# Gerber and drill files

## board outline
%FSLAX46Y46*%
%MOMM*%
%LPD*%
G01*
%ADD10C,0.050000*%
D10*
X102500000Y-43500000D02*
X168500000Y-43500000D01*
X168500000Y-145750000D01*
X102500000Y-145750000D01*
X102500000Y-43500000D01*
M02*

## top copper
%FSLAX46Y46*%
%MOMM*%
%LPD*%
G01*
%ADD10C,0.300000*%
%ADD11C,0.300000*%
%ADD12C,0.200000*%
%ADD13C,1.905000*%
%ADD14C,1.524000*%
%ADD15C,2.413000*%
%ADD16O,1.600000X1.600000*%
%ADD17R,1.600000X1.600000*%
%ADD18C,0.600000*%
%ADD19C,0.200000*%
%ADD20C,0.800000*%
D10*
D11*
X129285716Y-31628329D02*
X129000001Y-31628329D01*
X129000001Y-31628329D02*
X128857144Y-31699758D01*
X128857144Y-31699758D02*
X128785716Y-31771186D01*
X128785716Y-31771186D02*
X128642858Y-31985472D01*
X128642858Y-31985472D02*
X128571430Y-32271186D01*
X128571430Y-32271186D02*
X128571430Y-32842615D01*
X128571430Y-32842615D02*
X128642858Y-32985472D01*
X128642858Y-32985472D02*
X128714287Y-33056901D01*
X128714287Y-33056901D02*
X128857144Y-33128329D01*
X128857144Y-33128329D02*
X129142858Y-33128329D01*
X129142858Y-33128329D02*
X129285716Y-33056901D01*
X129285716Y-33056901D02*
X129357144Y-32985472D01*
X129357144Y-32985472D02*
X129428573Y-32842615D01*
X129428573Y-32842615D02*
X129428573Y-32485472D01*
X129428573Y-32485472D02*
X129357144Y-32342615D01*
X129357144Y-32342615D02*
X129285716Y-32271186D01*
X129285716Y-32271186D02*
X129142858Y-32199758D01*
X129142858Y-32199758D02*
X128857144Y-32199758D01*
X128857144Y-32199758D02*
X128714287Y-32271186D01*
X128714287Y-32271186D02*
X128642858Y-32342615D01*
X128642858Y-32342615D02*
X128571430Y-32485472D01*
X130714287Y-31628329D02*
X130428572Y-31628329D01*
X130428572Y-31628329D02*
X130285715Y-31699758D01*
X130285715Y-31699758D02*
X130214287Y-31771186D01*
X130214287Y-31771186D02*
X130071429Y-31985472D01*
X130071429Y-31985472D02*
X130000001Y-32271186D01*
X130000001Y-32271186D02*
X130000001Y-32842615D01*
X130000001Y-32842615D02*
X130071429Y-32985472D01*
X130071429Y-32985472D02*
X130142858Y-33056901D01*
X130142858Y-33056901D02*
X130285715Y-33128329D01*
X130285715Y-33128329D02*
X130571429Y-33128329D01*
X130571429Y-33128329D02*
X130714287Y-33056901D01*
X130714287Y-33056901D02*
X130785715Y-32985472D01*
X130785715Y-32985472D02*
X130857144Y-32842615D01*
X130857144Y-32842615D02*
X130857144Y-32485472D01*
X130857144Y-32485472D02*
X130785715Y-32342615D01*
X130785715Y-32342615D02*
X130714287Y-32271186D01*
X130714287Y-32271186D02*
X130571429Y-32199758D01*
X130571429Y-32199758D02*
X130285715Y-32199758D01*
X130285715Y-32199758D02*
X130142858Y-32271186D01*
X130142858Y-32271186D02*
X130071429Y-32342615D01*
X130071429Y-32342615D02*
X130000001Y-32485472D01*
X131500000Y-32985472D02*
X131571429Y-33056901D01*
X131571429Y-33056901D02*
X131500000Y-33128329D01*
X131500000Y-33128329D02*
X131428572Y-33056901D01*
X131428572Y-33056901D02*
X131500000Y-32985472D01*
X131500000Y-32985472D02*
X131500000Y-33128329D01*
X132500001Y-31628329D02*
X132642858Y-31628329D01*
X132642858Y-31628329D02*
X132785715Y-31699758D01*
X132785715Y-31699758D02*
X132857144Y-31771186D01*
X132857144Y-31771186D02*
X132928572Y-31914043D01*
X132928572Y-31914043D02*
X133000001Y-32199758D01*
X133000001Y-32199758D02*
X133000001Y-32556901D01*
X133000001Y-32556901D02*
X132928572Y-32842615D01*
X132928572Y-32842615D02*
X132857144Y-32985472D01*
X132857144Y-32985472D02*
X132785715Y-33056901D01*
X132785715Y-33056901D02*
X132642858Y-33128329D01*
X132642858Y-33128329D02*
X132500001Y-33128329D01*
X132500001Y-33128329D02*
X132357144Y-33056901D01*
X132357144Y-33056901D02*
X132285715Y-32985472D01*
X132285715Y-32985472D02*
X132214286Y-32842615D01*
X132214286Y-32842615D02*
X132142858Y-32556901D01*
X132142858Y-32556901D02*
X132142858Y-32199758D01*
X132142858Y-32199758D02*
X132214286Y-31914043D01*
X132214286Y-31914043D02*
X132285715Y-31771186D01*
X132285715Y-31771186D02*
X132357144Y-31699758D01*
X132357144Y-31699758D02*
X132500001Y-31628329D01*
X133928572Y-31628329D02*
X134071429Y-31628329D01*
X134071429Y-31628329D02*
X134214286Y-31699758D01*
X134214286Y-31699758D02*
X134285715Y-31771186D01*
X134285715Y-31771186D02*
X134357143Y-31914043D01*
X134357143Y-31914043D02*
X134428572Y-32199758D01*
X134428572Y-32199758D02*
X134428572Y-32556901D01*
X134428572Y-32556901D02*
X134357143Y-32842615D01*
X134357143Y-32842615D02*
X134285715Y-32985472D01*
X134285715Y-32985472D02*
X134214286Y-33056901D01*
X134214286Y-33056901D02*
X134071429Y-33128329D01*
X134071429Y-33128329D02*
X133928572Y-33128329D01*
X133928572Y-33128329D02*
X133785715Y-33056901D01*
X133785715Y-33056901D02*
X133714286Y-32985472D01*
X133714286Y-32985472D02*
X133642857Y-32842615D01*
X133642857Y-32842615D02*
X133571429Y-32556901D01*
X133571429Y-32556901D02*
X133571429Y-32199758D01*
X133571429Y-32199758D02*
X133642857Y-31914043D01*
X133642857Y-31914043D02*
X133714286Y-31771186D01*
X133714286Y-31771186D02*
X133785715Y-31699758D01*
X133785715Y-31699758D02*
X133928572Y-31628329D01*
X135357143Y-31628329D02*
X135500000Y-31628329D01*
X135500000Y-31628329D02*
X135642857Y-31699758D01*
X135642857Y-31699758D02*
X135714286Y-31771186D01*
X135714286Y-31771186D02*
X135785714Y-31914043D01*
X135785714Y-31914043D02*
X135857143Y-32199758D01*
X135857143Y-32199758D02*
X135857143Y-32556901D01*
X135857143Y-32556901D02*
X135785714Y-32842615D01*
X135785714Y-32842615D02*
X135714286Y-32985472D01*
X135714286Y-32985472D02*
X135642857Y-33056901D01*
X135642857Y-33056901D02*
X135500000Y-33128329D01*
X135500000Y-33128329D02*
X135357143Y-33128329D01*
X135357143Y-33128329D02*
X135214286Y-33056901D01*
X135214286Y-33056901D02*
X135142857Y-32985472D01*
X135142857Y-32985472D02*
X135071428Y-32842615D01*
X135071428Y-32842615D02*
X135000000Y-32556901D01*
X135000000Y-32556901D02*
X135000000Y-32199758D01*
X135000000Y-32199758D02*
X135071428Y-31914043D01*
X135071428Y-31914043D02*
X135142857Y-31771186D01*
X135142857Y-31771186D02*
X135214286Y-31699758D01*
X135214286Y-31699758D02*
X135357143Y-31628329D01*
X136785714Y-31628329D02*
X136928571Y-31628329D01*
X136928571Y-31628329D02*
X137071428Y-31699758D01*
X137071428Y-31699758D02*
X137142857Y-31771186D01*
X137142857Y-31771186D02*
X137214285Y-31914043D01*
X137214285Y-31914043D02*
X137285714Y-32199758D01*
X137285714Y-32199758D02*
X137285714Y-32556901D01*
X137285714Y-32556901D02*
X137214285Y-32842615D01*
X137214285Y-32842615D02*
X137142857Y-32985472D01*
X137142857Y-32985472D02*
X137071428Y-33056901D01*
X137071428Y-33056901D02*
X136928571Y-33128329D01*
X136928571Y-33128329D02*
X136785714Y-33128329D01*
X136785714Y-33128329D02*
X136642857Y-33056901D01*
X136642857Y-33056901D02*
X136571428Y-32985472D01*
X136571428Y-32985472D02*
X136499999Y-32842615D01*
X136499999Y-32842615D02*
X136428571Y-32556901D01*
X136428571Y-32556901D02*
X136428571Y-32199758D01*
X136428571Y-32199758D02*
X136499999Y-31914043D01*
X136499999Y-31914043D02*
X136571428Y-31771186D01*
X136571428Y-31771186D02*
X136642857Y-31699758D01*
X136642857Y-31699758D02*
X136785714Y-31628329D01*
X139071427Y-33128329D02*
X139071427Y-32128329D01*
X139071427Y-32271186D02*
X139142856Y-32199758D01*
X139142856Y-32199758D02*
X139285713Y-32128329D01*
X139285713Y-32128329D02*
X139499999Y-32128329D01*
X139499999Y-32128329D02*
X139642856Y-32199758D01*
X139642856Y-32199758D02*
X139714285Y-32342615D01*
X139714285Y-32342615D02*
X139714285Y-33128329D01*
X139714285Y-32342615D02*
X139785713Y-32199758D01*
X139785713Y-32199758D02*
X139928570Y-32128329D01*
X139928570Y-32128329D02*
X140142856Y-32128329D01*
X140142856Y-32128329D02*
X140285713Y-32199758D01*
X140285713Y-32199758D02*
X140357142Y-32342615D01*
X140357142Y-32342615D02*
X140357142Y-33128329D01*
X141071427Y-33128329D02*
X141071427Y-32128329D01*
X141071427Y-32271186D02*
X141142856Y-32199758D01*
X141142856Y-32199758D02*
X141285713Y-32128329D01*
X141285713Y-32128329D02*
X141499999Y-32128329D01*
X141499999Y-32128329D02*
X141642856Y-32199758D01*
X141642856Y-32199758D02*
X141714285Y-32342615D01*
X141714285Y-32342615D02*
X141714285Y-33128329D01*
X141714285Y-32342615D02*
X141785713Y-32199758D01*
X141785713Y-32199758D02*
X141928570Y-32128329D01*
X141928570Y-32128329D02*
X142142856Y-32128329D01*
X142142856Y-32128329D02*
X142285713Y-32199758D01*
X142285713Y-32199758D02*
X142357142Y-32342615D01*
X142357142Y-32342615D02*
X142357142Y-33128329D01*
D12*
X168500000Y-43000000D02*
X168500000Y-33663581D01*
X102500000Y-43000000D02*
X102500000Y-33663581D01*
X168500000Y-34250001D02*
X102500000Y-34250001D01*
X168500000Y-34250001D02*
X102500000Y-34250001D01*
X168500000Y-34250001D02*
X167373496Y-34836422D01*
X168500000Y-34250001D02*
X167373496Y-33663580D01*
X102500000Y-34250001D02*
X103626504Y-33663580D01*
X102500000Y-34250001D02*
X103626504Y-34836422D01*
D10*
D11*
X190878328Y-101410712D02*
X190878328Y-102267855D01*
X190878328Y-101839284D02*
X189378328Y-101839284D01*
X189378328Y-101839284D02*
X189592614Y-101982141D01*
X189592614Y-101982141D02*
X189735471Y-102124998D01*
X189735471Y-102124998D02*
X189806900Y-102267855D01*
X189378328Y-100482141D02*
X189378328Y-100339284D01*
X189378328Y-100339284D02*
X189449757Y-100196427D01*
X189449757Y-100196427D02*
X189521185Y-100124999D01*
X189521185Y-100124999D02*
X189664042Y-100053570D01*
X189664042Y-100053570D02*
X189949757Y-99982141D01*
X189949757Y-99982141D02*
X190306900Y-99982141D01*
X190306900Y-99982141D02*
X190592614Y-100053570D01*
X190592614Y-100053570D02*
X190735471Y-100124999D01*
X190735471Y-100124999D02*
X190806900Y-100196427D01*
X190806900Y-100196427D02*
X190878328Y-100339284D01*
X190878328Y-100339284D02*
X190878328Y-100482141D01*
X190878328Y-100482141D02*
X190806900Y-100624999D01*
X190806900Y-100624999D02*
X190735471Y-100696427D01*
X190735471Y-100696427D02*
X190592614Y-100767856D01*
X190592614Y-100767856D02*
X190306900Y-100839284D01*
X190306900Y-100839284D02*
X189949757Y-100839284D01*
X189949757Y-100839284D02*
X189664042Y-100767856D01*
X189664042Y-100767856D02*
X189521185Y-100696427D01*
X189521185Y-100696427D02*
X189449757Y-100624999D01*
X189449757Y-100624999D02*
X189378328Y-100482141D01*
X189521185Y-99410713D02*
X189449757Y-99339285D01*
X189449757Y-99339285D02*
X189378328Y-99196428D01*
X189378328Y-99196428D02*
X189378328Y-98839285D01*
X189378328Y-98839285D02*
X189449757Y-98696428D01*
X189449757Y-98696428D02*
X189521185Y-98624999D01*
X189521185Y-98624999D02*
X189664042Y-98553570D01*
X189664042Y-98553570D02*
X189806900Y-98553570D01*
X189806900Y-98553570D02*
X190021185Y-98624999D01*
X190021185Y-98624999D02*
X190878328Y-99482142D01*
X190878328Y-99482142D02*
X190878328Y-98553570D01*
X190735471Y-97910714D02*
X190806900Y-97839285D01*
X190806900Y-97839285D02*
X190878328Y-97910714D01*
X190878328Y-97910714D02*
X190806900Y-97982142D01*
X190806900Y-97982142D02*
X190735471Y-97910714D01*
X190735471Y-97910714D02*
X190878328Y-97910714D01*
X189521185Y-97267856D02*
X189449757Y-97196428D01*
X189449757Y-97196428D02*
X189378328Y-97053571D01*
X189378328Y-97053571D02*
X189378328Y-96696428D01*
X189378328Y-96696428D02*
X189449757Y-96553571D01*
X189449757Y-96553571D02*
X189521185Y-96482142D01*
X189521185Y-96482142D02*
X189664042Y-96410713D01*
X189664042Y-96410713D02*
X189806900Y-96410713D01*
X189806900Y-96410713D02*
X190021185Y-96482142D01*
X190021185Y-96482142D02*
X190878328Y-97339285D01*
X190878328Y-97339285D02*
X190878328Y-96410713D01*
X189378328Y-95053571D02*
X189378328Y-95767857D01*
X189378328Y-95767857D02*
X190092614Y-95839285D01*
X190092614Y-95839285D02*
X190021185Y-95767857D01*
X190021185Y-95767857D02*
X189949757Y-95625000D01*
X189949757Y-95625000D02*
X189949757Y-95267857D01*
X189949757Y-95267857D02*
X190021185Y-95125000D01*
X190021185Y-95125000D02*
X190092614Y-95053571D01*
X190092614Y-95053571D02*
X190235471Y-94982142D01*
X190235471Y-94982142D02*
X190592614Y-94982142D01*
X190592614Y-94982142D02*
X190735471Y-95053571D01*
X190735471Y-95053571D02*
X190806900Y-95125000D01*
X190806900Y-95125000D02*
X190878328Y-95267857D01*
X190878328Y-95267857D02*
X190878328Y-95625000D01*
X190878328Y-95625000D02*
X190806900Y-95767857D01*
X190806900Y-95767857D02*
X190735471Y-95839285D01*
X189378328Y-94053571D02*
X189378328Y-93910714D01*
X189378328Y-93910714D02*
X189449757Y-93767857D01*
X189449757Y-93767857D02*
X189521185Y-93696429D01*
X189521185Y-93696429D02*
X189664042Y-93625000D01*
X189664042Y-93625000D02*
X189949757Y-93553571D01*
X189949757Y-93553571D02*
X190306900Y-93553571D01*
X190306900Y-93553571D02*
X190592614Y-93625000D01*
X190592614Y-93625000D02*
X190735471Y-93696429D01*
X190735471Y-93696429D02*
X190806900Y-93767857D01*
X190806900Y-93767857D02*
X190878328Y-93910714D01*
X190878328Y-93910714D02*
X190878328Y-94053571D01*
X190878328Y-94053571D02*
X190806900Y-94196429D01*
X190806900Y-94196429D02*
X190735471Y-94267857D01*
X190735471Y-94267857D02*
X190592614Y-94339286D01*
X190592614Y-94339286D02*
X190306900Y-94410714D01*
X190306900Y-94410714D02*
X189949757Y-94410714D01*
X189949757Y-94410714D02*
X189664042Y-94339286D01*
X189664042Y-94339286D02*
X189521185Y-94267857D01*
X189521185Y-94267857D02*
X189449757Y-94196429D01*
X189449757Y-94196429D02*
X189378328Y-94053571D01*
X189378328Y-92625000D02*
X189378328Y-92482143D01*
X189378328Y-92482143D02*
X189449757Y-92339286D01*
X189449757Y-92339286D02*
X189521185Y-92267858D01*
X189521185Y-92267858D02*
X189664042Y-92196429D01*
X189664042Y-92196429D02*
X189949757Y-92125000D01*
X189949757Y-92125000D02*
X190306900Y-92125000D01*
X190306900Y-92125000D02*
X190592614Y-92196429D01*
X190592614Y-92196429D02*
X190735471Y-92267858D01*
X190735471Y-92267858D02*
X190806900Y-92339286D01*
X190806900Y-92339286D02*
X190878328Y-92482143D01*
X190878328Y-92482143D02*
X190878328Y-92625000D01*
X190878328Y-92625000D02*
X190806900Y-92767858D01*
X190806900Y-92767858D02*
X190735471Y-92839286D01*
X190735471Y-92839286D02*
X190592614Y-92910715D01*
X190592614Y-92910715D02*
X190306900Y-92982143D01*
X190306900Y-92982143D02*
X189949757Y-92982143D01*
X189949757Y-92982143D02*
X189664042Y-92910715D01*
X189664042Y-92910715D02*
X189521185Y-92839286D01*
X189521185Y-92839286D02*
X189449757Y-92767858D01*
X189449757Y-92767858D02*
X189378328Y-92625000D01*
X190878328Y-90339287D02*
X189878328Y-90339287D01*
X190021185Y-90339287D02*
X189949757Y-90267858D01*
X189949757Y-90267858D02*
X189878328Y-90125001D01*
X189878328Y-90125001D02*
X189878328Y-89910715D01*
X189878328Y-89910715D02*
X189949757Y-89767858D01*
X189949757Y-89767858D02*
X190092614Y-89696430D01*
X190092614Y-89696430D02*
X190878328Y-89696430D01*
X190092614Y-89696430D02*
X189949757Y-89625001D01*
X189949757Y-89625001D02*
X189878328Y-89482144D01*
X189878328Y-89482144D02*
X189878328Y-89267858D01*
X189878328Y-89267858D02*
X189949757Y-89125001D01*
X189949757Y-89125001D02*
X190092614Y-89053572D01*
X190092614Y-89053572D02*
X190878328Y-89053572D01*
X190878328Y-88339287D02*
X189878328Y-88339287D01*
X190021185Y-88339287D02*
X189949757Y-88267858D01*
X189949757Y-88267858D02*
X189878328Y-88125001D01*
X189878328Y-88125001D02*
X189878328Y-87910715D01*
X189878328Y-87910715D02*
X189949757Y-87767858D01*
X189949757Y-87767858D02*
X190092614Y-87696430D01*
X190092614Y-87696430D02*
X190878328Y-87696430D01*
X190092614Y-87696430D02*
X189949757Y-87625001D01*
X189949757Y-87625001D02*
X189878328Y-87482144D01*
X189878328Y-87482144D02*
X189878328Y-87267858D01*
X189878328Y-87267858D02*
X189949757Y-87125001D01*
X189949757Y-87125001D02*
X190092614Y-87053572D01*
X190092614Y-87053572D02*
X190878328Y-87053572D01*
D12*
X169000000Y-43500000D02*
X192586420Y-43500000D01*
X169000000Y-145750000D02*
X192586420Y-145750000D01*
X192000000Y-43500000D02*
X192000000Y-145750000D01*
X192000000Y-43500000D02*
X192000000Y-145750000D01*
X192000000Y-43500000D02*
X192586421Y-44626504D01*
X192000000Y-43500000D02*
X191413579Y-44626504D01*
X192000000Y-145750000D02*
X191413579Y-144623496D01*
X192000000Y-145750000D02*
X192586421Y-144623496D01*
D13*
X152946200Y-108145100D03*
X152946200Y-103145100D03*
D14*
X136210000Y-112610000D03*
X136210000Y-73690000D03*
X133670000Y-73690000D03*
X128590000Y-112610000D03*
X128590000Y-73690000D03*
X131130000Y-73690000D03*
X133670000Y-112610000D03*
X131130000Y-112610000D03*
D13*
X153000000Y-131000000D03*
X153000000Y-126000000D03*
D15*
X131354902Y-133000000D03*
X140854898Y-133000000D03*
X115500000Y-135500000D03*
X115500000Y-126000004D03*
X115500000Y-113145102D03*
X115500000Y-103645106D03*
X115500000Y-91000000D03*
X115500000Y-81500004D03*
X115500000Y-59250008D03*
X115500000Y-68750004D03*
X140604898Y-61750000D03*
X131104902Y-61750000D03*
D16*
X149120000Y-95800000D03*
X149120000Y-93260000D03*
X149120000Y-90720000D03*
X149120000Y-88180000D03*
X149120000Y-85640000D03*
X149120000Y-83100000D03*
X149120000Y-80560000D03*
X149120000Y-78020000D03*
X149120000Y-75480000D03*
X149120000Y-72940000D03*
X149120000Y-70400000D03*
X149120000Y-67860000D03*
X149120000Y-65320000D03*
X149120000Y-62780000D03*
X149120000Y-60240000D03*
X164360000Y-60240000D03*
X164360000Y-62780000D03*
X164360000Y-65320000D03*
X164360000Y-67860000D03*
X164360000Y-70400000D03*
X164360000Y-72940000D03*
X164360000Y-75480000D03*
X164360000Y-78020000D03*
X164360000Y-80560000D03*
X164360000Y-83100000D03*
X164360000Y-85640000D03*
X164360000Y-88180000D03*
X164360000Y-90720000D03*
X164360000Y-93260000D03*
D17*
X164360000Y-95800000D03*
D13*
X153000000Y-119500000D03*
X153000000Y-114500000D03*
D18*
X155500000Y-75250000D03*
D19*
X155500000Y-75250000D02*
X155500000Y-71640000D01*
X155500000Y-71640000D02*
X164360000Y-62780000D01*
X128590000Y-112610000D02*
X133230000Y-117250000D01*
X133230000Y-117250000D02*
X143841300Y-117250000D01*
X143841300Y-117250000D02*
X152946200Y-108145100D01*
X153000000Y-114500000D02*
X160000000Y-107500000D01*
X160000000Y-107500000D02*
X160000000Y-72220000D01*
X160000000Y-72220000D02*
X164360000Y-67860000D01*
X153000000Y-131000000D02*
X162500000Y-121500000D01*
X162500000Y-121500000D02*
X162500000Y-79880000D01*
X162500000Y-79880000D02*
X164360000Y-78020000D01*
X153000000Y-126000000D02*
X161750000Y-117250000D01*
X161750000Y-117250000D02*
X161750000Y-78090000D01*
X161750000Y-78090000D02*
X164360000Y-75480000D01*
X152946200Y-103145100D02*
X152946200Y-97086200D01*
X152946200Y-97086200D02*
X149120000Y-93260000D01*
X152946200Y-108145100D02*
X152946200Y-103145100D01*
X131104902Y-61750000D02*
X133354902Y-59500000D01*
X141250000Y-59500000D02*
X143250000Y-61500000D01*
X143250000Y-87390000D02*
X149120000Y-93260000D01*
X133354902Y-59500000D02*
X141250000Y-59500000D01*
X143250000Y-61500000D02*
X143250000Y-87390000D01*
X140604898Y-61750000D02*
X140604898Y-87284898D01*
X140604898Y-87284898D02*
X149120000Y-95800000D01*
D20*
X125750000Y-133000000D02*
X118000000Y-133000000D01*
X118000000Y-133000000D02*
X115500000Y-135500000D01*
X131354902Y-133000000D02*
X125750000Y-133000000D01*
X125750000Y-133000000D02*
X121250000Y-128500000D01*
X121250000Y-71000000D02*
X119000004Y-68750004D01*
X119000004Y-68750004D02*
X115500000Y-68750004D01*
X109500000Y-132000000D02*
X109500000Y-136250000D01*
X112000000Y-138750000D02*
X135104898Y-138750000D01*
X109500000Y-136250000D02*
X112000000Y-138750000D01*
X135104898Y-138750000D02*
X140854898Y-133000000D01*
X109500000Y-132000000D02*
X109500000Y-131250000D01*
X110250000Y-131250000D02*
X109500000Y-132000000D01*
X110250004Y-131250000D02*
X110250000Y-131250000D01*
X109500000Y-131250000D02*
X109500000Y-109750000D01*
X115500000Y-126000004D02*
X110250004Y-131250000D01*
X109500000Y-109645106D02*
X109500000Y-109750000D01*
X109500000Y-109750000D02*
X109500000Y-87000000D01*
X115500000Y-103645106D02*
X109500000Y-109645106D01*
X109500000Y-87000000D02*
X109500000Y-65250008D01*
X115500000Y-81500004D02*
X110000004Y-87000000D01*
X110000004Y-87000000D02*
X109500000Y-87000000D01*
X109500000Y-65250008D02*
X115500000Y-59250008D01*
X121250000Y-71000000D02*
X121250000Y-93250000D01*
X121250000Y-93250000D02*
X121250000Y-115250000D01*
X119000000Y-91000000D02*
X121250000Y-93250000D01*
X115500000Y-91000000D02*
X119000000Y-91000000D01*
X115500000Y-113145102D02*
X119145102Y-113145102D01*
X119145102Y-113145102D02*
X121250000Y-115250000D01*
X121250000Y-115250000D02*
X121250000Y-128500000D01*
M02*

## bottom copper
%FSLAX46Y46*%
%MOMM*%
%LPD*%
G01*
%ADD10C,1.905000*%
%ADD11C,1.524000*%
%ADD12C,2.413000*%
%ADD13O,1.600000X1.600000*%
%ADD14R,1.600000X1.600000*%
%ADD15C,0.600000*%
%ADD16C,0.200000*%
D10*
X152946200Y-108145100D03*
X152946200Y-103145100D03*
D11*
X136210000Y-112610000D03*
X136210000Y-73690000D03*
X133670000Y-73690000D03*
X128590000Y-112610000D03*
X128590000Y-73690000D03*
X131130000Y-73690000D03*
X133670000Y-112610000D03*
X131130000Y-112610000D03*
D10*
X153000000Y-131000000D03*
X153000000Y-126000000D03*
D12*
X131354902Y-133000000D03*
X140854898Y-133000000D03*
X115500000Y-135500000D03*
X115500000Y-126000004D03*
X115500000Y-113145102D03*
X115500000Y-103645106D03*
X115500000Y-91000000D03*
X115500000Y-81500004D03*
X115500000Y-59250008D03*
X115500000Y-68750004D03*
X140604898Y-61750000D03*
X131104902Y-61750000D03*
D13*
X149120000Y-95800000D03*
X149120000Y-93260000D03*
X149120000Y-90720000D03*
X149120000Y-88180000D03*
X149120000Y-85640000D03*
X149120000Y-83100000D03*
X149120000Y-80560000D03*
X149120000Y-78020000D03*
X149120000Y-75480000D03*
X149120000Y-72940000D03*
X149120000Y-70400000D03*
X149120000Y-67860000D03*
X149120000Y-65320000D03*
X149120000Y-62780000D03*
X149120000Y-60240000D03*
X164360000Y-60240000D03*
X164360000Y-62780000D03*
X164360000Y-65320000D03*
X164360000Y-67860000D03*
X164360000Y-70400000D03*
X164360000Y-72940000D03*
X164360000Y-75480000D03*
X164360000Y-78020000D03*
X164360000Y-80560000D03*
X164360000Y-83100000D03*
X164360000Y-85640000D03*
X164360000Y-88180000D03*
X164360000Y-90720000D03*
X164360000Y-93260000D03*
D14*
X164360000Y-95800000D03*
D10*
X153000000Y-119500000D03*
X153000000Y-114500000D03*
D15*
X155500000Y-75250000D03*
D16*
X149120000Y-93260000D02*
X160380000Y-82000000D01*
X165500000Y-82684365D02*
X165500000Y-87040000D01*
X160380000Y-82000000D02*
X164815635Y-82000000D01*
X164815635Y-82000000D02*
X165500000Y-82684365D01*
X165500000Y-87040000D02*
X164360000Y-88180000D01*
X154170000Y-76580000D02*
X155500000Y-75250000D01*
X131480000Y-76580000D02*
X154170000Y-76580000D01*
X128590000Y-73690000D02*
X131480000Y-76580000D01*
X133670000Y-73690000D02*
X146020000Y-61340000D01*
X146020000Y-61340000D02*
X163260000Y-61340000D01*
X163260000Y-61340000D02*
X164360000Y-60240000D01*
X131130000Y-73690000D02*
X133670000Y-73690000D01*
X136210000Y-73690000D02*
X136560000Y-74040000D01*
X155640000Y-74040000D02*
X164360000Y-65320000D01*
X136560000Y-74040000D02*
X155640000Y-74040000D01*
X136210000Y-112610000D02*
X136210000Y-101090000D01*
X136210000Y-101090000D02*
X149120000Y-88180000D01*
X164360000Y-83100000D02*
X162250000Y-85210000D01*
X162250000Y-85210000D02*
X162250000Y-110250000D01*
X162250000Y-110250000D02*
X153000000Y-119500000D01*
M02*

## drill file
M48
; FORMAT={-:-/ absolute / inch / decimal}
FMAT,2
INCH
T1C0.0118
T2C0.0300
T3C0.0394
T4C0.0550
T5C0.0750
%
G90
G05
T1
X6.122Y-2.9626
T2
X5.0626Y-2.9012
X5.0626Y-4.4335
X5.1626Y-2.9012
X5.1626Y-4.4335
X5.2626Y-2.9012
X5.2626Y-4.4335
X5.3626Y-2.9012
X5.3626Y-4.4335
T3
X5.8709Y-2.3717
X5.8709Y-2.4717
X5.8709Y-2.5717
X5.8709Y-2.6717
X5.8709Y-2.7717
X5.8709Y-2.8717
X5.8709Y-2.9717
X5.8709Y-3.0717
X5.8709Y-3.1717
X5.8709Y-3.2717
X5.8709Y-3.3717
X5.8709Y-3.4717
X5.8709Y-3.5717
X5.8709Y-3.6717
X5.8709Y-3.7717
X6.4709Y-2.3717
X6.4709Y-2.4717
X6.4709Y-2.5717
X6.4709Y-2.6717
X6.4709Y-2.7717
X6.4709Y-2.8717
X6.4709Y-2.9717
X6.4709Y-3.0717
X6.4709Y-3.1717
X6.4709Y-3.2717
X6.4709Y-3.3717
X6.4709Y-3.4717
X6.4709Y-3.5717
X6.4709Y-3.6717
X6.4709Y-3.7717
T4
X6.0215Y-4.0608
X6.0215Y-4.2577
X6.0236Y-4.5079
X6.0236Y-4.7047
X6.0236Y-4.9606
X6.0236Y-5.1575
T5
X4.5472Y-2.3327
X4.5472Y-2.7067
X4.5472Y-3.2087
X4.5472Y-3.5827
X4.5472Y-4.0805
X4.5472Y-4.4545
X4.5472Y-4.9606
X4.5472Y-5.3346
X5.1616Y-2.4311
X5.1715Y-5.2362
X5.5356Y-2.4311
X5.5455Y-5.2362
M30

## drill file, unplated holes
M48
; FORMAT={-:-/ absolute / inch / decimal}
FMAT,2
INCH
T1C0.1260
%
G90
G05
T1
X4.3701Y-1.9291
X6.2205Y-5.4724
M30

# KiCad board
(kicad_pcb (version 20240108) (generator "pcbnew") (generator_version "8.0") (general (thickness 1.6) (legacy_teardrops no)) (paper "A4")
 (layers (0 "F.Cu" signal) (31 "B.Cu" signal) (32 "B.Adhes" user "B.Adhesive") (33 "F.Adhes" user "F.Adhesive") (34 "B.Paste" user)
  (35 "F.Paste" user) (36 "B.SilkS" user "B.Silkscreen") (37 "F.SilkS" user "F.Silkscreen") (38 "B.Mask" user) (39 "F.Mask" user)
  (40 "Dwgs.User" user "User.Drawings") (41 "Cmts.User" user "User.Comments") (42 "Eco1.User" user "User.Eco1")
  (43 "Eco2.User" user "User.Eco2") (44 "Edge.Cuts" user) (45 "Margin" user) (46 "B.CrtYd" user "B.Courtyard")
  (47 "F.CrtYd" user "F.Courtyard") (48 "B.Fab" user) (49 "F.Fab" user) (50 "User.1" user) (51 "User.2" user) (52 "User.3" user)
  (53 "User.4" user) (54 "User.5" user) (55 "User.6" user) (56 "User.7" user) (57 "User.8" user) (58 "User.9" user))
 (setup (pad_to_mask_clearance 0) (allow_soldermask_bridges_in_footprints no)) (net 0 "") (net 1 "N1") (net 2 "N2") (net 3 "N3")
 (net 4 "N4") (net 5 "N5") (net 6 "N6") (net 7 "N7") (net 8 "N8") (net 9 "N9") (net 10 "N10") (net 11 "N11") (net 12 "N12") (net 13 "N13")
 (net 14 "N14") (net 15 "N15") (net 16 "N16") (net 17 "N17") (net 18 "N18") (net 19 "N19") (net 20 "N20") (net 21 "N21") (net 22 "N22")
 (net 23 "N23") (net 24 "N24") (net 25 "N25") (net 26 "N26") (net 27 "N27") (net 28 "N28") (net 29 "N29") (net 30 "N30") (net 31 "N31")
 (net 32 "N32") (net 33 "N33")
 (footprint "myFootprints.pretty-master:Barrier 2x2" (layer "F.Cu") (at 115.5 68.750004 90)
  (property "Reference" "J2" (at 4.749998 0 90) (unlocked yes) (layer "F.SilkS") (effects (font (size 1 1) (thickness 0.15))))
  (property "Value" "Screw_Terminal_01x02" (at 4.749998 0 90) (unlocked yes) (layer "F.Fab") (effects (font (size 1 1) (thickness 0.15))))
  (pad "1" thru_hole circle (at 0 0 90) (size 2.413 2.413) (drill 1.905) (layers "*.Cu" "*.Mask") (remove_unused_layers no) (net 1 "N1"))
  (pad "2" thru_hole circle (at 9.499996 0 90) (size 2.413 2.413) (drill 1.905) (layers "*.Cu" "*.Mask") (remove_unused_layers no)
   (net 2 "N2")))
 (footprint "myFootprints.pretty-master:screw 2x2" (layer "F.Cu") (at 153 119.5 90)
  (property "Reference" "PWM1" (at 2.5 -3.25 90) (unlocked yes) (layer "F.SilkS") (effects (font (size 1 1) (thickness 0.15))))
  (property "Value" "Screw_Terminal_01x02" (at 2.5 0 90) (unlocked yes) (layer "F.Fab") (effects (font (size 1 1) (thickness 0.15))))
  (pad "1" thru_hole circle (at 0 0 90) (size 1.905 1.905) (drill 1.397) (layers "*.Cu" "*.Mask") (remove_unused_layers no) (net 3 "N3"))
  (pad "2" thru_hole circle (at 5 0 90) (size 1.905 1.905) (drill 1.397) (layers "*.Cu" "*.Mask") (remove_unused_layers no) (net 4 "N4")))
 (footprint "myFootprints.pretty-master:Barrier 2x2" (layer "F.Cu") (at 131.354902 133)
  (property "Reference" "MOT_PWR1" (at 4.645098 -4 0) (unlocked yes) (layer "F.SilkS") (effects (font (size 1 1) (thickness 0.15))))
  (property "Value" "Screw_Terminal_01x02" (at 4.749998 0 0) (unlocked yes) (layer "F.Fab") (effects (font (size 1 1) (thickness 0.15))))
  (pad "1" thru_hole circle (at 0 0) (size 2.413 2.413) (drill 1.905) (layers "*.Cu" "*.Mask") (remove_unused_layers no) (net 1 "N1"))
  (pad "2" thru_hole circle (at 9.499996 0) (size 2.413 2.413) (drill 1.905) (layers "*.Cu" "*.Mask") (remove_unused_layers no) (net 2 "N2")))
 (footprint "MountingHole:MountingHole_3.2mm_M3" (layer "F.Cu") (at 111 49)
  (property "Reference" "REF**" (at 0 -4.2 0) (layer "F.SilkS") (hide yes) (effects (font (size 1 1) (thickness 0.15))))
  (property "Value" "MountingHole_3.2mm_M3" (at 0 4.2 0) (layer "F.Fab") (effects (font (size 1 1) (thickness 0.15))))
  (pad "" np_thru_hole circle (at 0 0) (size 3.2 3.2) (drill 3.2) (layers "*.Cu" "*.Mask")))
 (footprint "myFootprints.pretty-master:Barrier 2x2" (layer "F.Cu") (at 115.5 113.145102 90)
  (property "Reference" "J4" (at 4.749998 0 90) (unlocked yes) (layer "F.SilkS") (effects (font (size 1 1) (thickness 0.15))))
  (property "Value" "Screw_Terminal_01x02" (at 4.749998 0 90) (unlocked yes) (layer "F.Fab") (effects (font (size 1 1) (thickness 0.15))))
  (pad "1" thru_hole circle (at 0 0 90) (size 2.413 2.413) (drill 1.905) (layers "*.Cu" "*.Mask") (remove_unused_layers no) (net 1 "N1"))
  (pad "2" thru_hole circle (at 9.499996 0 90) (size 2.413 2.413) (drill 1.905) (layers "*.Cu" "*.Mask") (remove_unused_layers no)
   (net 2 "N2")))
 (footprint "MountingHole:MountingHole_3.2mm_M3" (layer "F.Cu") (at 158 139)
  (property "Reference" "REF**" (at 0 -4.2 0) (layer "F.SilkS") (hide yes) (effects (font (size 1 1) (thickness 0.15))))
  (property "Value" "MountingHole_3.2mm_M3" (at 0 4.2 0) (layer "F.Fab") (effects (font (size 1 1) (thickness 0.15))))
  (pad "" np_thru_hole circle (at 0 0) (size 3.2 3.2) (drill 3.2) (layers "F&B.Cu" "*.Mask")))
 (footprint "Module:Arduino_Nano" (layer "F.Cu") (at 164.36 95.8 180)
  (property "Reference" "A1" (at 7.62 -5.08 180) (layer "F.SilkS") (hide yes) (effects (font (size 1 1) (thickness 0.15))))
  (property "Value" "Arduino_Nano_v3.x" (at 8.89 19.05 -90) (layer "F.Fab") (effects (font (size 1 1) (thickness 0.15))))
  (pad "1" thru_hole rect (at 0 0 180) (size 1.6 1.6) (drill 1) (layers "*.Cu" "*.Mask") (remove_unused_layers no) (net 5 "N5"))
  (pad "2" thru_hole oval (at 0 2.54 180) (size 1.6 1.6) (drill 1) (layers "*.Cu" "*.Mask") (remove_unused_layers no) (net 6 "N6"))
  (pad "3" thru_hole oval (at 0 5.08 180) (size 1.6 1.6) (drill 1) (layers "*.Cu" "*.Mask") (remove_unused_layers no) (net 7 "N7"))
  (pad "4" thru_hole oval (at 0 7.62 180) (size 1.6 1.6) (drill 1) (layers "*.Cu" "*.Mask") (remove_unused_layers no) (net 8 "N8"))
  (pad "5" thru_hole oval (at 0 10.16 180) (size 1.6 1.6) (drill 1) (layers "*.Cu" "*.Mask") (remove_unused_layers no) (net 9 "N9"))
  (pad "6" thru_hole oval (at 0 12.7 180) (size 1.6 1.6) (drill 1) (layers "*.Cu" "*.Mask") (remove_unused_layers no) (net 3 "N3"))
  (pad "7" thru_hole oval (at 0 15.24 180) (size 1.6 1.6) (drill 1) (layers "*.Cu" "*.Mask") (remove_unused_layers no) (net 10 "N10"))
  (pad "8" thru_hole oval (at 0 17.78 180) (size 1.6 1.6) (drill 1) (layers "*.Cu" "*.Mask") (remove_unused_layers no) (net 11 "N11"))
  (pad "9" thru_hole oval (at 0 20.32 180) (size 1.6 1.6) (drill 1) (layers "*.Cu" "*.Mask") (remove_unused_layers no) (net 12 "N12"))
  (pad "10" thru_hole oval (at 0 22.86 180) (size 1.6 1.6) (drill 1) (layers "*.Cu" "*.Mask") (remove_unused_layers no) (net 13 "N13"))
  (pad "11" thru_hole oval (at 0 25.4 180) (size 1.6 1.6) (drill 1) (layers "*.Cu" "*.Mask") (remove_unused_layers no) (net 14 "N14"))
  (pad "12" thru_hole oval (at 0 27.94 180) (size 1.6 1.6) (drill 1) (layers "*.Cu" "*.Mask") (remove_unused_layers no) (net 4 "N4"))
  (pad "13" thru_hole oval (at 0 30.48 180) (size 1.6 1.6) (drill 1) (layers "*.Cu" "*.Mask") (remove_unused_layers no) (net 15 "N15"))
  (pad "14" thru_hole oval (at 0 33.02 180) (size 1.6 1.6) (drill 1) (layers "*.Cu" "*.Mask") (remove_unused_layers no) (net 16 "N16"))
  (pad "15" thru_hole oval (at 0 35.56 180) (size 1.6 1.6) (drill 1) (layers "*.Cu" "*.Mask") (remove_unused_layers no) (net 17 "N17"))
  (pad "16" thru_hole oval (at 15.24 35.56 180) (size 1.6 1.6) (drill 1) (layers "*.Cu" "*.Mask") (remove_unused_layers no) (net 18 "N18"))
  (pad "17" thru_hole oval (at 15.24 33.02 180) (size 1.6 1.6) (drill 1) (layers "*.Cu" "*.Mask") (remove_unused_layers no) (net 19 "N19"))
  (pad "18" thru_hole oval (at 15.24 30.48 180) (size 1.6 1.6) (drill 1) (layers "*.Cu" "*.Mask") (remove_unused_layers no) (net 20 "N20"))
  (pad "19" thru_hole oval (at 15.24 27.94 180) (size 1.6 1.6) (drill 1) (layers "*.Cu" "*.Mask") (remove_unused_layers no) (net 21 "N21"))
  (pad "20" thru_hole oval (at 15.24 25.4 180) (size 1.6 1.6) (drill 1) (layers "*.Cu" "*.Mask") (remove_unused_layers no) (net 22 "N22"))
  (pad "21" thru_hole oval (at 15.24 22.86 180) (size 1.6 1.6) (drill 1) (layers "*.Cu" "*.Mask") (remove_unused_layers no) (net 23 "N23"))
  (pad "22" thru_hole oval (at 15.24 20.32 180) (size 1.6 1.6) (drill 1) (layers "*.Cu" "*.Mask") (remove_unused_layers no) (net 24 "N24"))
  (pad "23" thru_hole oval (at 15.24 17.78 180) (size 1.6 1.6) (drill 1) (layers "*.Cu" "*.Mask") (remove_unused_layers no) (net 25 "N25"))
  (pad "24" thru_hole oval (at 15.24 15.24 180) (size 1.6 1.6) (drill 1) (layers "*.Cu" "*.Mask") (remove_unused_layers no) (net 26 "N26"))
  (pad "25" thru_hole oval (at 15.24 12.7 180) (size 1.6 1.6) (drill 1) (layers "*.Cu" "*.Mask") (remove_unused_layers no) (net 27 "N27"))
  (pad "26" thru_hole oval (at 15.24 10.16 180) (size 1.6 1.6) (drill 1) (layers "*.Cu" "*.Mask") (remove_unused_layers no) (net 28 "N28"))
  (pad "27" thru_hole oval (at 15.24 7.62 180) (size 1.6 1.6) (drill 1) (layers "*.Cu" "*.Mask") (remove_unused_layers no) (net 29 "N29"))
  (pad "28" thru_hole oval (at 15.24 5.08 180) (size 1.6 1.6) (drill 1) (layers "*.Cu" "*.Mask") (remove_unused_layers no) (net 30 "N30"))
  (pad "29" thru_hole oval (at 15.24 2.54 180) (size 1.6 1.6) (drill 1) (layers "*.Cu" "*.Mask") (remove_unused_layers no) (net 8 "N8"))
  (pad "30" thru_hole oval (at 15.24 0 180) (size 1.6 1.6) (drill 1) (layers "*.Cu" "*.Mask") (remove_unused_layers no) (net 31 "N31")))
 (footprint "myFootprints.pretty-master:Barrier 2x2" (layer "F.Cu") (at 115.5 135.5 90)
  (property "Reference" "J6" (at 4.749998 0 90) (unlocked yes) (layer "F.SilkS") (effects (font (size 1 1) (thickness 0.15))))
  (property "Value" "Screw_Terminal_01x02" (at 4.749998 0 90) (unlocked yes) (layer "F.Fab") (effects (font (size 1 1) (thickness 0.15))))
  (pad "1" thru_hole circle (at 0 0 90) (size 2.413 2.413) (drill 1.905) (layers "*.Cu" "*.Mask") (remove_unused_layers no) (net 1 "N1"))
  (pad "2" thru_hole circle (at 9.499996 0 90) (size 2.413 2.413) (drill 1.905) (layers "*.Cu" "*.Mask") (remove_unused_layers no)
   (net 2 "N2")))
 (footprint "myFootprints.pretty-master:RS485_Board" (layer "F.Cu") (at 139.4 115.15 -90)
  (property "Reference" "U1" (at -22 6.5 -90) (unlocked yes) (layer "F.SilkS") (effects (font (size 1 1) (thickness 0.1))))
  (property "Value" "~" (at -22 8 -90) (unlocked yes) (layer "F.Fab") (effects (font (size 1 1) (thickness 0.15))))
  (pad "A" thru_hole circle (at -2.54 8.27 270) (size 1.524 1.524) (drill 0.762) (layers "*.Cu" "*.Mask") (remove_unused_layers no)
   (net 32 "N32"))
  (pad "B" thru_hole circle (at -2.54 5.73 270) (size 1.524 1.524) (drill 0.762) (layers "*.Cu" "*.Mask") (remove_unused_layers no)
   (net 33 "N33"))
  (pad "DE" thru_hole circle (at -41.46 8.27 270) (size 1.524 1.524) (drill 0.762) (layers "*.Cu" "*.Mask") (remove_unused_layers no)
   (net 17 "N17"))
  (pad "DI" thru_hole circle (at -41.46 10.81 270) (size 1.524 1.524) (drill 0.762) (layers "*.Cu" "*.Mask") (remove_unused_layers no)
   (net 16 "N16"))
  (pad "GND" thru_hole circle (at -2.54 10.81 270) (size 1.524 1.524) (drill 0.762) (layers "*.Cu" "*.Mask") (remove_unused_layers no)
   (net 8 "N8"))
  (pad "RE" thru_hole circle (at -41.46 5.73 270) (size 1.524 1.524) (drill 0.762) (layers "*.Cu" "*.Mask") (remove_unused_layers no)
   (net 17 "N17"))
  (pad "RO" thru_hole circle (at -41.46 3.19 270) (size 1.524 1.524) (drill 0.762) (layers "*.Cu" "*.Mask") (remove_unused_layers no)
   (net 15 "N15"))
  (pad "VCC" thru_hole circle (at -2.54 3.19 270) (size 1.524 1.524) (drill 0.762) (layers "*.Cu" "*.Mask") (remove_unused_layers no)
   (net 29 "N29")))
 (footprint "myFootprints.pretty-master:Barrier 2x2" (layer "F.Cu") (at 131.104902 61.75)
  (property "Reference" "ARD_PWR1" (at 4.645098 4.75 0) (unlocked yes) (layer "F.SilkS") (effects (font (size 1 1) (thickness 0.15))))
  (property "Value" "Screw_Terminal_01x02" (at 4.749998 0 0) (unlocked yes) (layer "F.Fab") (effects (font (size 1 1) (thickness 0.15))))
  (pad "1" thru_hole circle (at 0 0) (size 2.413 2.413) (drill 1.905) (layers "*.Cu" "*.Mask") (remove_unused_layers no) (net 8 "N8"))
  (pad "2" thru_hole circle (at 9.499996 0) (size 2.413 2.413) (drill 1.905) (layers "*.Cu" "*.Mask") (remove_unused_layers no)
   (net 31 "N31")))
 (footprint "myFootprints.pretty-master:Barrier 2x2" (layer "F.Cu") (at 115.5 91 90)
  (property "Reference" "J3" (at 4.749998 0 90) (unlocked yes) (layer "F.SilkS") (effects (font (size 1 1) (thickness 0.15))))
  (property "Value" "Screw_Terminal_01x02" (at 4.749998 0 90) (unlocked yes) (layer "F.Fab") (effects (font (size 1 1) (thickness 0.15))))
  (pad "1" thru_hole circle (at 0 0 90) (size 2.413 2.413) (drill 1.905) (layers "*.Cu" "*.Mask") (remove_unused_layers no) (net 1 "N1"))
  (pad "2" thru_hole circle (at 9.499996 0 90) (size 2.413 2.413) (drill 1.905) (layers "*.Cu" "*.Mask") (remove_unused_layers no)
   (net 2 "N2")))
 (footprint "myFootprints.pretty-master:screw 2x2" (layer "F.Cu") (at 153 131 90)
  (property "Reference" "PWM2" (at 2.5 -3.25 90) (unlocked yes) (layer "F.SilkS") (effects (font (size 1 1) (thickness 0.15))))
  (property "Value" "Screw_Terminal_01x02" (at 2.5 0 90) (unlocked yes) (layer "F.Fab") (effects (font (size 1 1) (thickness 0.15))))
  (pad "1" thru_hole circle (at 0 0 90) (size 1.905 1.905) (drill 1.397) (layers "*.Cu" "*.Mask") (remove_unused_layers no) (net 11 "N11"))
  (pad "2" thru_hole circle (at 5 0 90) (size 1.905 1.905) (drill 1.397) (layers "*.Cu" "*.Mask") (remove_unused_layers no) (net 12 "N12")))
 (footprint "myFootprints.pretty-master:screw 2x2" (layer "F.Cu") (at 152.9462 108.1451 90)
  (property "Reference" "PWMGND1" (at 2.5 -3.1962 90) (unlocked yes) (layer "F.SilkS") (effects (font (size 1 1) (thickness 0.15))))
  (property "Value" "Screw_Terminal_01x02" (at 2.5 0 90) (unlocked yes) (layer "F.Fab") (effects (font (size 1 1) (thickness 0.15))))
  (pad "1" thru_hole circle (at 0 0 90) (size 1.905 1.905) (drill 1.397) (layers "*.Cu" "*.Mask") (remove_unused_layers no) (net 8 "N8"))
  (pad "2" thru_hole circle (at 5 0 90) (size 1.905 1.905) (drill 1.397) (layers "*.Cu" "*.Mask") (remove_unused_layers no) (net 8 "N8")))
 (gr_rect (start 102.5 43.5) (end 168.5 145.75) (stroke (width 0.05) (type default)) (fill none) (layer "Edge.Cuts"))
 (segment (start 155.5 71.64) (end 164.36 62.78) (width 0.2) (layer "F.Cu") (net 16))
 (segment (start 155.5 75.25) (end 155.5 71.64) (width 0.2) (layer "F.Cu") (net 16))
 (via (at 155.5 75.25) (size 0.6) (drill 0.3) (layers "F.Cu" "B.Cu") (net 16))
 (segment (start 131.48 76.58) (end 154.17 76.58) (width 0.2) (layer "B.Cu") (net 16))
 (segment (start 154.17 76.58) (end 155.5 75.25) (width 0.2) (layer "B.Cu") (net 16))
 (segment (start 128.59 73.69) (end 131.48 76.58) (width 0.2) (layer "B.Cu") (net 16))
 (segment (start 140.604898 87.284898) (end 149.12 95.8) (width 0.2) (layer "F.Cu") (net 31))
 (segment (start 140.604898 61.75) (end 140.604898 87.284898) (width 0.2) (layer "F.Cu") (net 31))
 (segment (start 131.104902 61.75) (end 133.354902 59.5) (width 0.2) (layer "F.Cu") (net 8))
 (segment (start 152.9462 97.0862) (end 149.12 93.26) (width 0.2) (layer "F.Cu") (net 8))
 (segment (start 143.25 87.39) (end 149.12 93.26) (width 0.2) (layer "F.Cu") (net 8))
 (segment (start 143.8413 117.25) (end 152.9462 108.1451) (width 0.2) (layer "F.Cu") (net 8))
 (segment (start 141.25 59.5) (end 143.25 61.5) (width 0.2) (layer "F.Cu") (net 8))
 (segment (start 133.354902 59.5) (end 141.25 59.5) (width 0.2) (layer "F.Cu") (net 8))
 (segment (start 152.9462 108.1451) (end 152.9462 103.1451) (width 0.2) (layer "F.Cu") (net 8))
 (segment (start 143.25 61.5) (end 143.25 87.39) (width 0.2) (layer "F.Cu") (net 8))
 (segment (start 128.59 112.61) (end 133.23 117.25) (width 0.2) (layer "F.Cu") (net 8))
 (segment (start 152.9462 103.1451) (end 152.9462 97.0862) (width 0.2) (layer "F.Cu") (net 8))
 (segment (start 133.23 117.25) (end 143.8413 117.25) (width 0.2) (layer "F.Cu") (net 8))
 (segment (start 149.12 93.26) (end 160.38 82) (width 0.2) (layer "B.Cu") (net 8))
 (segment (start 160.38 82) (end 164.815635 82) (width 0.2) (layer "B.Cu") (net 8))
 (segment (start 164.815635 82) (end 165.5 82.684365) (width 0.2) (layer "B.Cu") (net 8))
 (segment (start 165.5 82.684365) (end 165.5 87.04) (width 0.2) (layer "B.Cu") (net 8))
 (segment (start 165.5 87.04) (end 164.36 88.18) (width 0.2) (layer "B.Cu") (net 8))
 (segment (start 136.56 74.04) (end 155.64 74.04) (width 0.2) (layer "B.Cu") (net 15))
 (segment (start 155.64 74.04) (end 164.36 65.32) (width 0.2) (layer "B.Cu") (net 15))
 (segment (start 136.21 73.69) (end 136.56 74.04) (width 0.2) (layer "B.Cu") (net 15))
 (segment (start 163.26 61.34) (end 164.36 60.24) (width 0.2) (layer "B.Cu") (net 17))
 (segment (start 146.02 61.34) (end 163.26 61.34) (width 0.2) (layer "B.Cu") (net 17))
 (segment (start 133.67 73.69) (end 146.02 61.34) (width 0.2) (layer "B.Cu") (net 17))
 (segment (start 131.13 73.69) (end 133.67 73.69) (width 0.2) (layer "B.Cu") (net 17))
 (segment (start 153 126) (end 161.75 117.25) (width 0.2) (layer "F.Cu") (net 12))
 (segment (start 161.75 78.09) (end 164.36 75.48) (width 0.2) (layer "F.Cu") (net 12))
 (segment (start 161.75 117.25) (end 161.75 78.09) (width 0.2) (layer "F.Cu") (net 12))
 (segment (start 160 72.22) (end 164.36 67.86) (width 0.2) (layer "F.Cu") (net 4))
 (segment (start 160 107.5) (end 160 72.22) (width 0.2) (layer "F.Cu") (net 4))
 (segment (start 153 114.5) (end 160 107.5) (width 0.2) (layer "F.Cu") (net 4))
 (segment (start 153 131) (end 162.5 121.5) (width 0.2) (layer "F.Cu") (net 11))
 (segment (start 162.5 121.5) (end 162.5 79.88) (width 0.2) (layer "F.Cu") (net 11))
 (segment (start 162.5 79.88) (end 164.36 78.02) (width 0.2) (layer "F.Cu") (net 11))
 (segment (start 162.25 85.21) (end 162.25 110.25) (width 0.2) (layer "B.Cu") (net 3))
 (segment (start 162.25 110.25) (end 153 119.5) (width 0.2) (layer "B.Cu") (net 3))
 (segment (start 164.36 83.1) (end 162.25 85.21) (width 0.2) (layer "B.Cu") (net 3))
 (segment (start 110.250004 131.25) (end 110.25 131.25) (width 0.8) (layer "F.Cu") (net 2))
 (segment (start 112 138.75) (end 135.104898 138.75) (width 0.8) (layer "F.Cu") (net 2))
 (segment (start 109.5 131.25) (end 109.5 109.75) (width 0.8) (layer "F.Cu") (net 2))
 (segment (start 115.5 81.500004) (end 110.000004 87) (width 0.8) (layer "F.Cu") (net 2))
 (segment (start 109.5 65.250008) (end 115.5 59.250008) (width 0.8) (layer "F.Cu") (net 2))
 (segment (start 115.5 103.645106) (end 109.5 109.645106) (width 0.8) (layer "F.Cu") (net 2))
 (segment (start 109.5 109.75) (end 109.5 87) (width 0.8) (layer "F.Cu") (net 2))
 (segment (start 109.5 132) (end 109.5 131.25) (width 0.8) (layer "F.Cu") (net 2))
 (segment (start 135.104898 138.75) (end 140.854898 133) (width 0.8) (layer "F.Cu") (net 2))
 (segment (start 109.5 132) (end 109.5 136.25) (width 0.8) (layer "F.Cu") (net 2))
 (segment (start 110.25 131.25) (end 109.5 132) (width 0.8) (layer "F.Cu") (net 2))
 (segment (start 109.5 136.25) (end 112 138.75) (width 0.8) (layer "F.Cu") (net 2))
 (segment (start 110.000004 87) (end 109.5 87) (width 0.8) (layer "F.Cu") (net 2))
 (segment (start 115.5 126.000004) (end 110.250004 131.25) (width 0.8) (layer "F.Cu") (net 2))
 (segment (start 109.5 87) (end 109.5 65.250008) (width 0.8) (layer "F.Cu") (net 2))
 (segment (start 109.5 109.645106) (end 109.5 109.75) (width 0.8) (layer "F.Cu") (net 2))
 (segment (start 125.75 133) (end 118 133) (width 0.8) (layer "F.Cu") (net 1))
 (segment (start 125.75 133) (end 121.25 128.5) (width 0.8) (layer "F.Cu") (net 1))
 (segment (start 121.25 71) (end 119.000004 68.750004) (width 0.8) (layer "F.Cu") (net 1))
 (segment (start 119.000004 68.750004) (end 115.5 68.750004) (width 0.8) (layer "F.Cu") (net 1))
 (segment (start 131.354902 133) (end 125.75 133) (width 0.8) (layer "F.Cu") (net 1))
 (segment (start 119.145102 113.145102) (end 121.25 115.25) (width 0.8) (layer "F.Cu") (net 1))
 (segment (start 121.25 115.25) (end 121.25 128.5) (width 0.8) (layer "F.Cu") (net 1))
 (segment (start 115.5 91) (end 119 91) (width 0.8) (layer "F.Cu") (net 1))
 (segment (start 121.25 71) (end 121.25 93.25) (width 0.8) (layer "F.Cu") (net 1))
 (segment (start 121.25 93.25) (end 121.25 115.25) (width 0.8) (layer "F.Cu") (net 1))
 (segment (start 115.5 113.145102) (end 119.145102 113.145102) (width 0.8) (layer "F.Cu") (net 1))
 (segment (start 119 91) (end 121.25 93.25) (width 0.8) (layer "F.Cu") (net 1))
 (segment (start 118 133) (end 115.5 135.5) (width 0.8) (layer "F.Cu") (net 1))
 (segment (start 136.21 101.09) (end 149.12 88.18) (width 0.2) (layer "B.Cu") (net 29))
 (segment (start 136.21 112.61) (end 136.21 101.09) (width 0.2) (layer "B.Cu") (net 29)))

